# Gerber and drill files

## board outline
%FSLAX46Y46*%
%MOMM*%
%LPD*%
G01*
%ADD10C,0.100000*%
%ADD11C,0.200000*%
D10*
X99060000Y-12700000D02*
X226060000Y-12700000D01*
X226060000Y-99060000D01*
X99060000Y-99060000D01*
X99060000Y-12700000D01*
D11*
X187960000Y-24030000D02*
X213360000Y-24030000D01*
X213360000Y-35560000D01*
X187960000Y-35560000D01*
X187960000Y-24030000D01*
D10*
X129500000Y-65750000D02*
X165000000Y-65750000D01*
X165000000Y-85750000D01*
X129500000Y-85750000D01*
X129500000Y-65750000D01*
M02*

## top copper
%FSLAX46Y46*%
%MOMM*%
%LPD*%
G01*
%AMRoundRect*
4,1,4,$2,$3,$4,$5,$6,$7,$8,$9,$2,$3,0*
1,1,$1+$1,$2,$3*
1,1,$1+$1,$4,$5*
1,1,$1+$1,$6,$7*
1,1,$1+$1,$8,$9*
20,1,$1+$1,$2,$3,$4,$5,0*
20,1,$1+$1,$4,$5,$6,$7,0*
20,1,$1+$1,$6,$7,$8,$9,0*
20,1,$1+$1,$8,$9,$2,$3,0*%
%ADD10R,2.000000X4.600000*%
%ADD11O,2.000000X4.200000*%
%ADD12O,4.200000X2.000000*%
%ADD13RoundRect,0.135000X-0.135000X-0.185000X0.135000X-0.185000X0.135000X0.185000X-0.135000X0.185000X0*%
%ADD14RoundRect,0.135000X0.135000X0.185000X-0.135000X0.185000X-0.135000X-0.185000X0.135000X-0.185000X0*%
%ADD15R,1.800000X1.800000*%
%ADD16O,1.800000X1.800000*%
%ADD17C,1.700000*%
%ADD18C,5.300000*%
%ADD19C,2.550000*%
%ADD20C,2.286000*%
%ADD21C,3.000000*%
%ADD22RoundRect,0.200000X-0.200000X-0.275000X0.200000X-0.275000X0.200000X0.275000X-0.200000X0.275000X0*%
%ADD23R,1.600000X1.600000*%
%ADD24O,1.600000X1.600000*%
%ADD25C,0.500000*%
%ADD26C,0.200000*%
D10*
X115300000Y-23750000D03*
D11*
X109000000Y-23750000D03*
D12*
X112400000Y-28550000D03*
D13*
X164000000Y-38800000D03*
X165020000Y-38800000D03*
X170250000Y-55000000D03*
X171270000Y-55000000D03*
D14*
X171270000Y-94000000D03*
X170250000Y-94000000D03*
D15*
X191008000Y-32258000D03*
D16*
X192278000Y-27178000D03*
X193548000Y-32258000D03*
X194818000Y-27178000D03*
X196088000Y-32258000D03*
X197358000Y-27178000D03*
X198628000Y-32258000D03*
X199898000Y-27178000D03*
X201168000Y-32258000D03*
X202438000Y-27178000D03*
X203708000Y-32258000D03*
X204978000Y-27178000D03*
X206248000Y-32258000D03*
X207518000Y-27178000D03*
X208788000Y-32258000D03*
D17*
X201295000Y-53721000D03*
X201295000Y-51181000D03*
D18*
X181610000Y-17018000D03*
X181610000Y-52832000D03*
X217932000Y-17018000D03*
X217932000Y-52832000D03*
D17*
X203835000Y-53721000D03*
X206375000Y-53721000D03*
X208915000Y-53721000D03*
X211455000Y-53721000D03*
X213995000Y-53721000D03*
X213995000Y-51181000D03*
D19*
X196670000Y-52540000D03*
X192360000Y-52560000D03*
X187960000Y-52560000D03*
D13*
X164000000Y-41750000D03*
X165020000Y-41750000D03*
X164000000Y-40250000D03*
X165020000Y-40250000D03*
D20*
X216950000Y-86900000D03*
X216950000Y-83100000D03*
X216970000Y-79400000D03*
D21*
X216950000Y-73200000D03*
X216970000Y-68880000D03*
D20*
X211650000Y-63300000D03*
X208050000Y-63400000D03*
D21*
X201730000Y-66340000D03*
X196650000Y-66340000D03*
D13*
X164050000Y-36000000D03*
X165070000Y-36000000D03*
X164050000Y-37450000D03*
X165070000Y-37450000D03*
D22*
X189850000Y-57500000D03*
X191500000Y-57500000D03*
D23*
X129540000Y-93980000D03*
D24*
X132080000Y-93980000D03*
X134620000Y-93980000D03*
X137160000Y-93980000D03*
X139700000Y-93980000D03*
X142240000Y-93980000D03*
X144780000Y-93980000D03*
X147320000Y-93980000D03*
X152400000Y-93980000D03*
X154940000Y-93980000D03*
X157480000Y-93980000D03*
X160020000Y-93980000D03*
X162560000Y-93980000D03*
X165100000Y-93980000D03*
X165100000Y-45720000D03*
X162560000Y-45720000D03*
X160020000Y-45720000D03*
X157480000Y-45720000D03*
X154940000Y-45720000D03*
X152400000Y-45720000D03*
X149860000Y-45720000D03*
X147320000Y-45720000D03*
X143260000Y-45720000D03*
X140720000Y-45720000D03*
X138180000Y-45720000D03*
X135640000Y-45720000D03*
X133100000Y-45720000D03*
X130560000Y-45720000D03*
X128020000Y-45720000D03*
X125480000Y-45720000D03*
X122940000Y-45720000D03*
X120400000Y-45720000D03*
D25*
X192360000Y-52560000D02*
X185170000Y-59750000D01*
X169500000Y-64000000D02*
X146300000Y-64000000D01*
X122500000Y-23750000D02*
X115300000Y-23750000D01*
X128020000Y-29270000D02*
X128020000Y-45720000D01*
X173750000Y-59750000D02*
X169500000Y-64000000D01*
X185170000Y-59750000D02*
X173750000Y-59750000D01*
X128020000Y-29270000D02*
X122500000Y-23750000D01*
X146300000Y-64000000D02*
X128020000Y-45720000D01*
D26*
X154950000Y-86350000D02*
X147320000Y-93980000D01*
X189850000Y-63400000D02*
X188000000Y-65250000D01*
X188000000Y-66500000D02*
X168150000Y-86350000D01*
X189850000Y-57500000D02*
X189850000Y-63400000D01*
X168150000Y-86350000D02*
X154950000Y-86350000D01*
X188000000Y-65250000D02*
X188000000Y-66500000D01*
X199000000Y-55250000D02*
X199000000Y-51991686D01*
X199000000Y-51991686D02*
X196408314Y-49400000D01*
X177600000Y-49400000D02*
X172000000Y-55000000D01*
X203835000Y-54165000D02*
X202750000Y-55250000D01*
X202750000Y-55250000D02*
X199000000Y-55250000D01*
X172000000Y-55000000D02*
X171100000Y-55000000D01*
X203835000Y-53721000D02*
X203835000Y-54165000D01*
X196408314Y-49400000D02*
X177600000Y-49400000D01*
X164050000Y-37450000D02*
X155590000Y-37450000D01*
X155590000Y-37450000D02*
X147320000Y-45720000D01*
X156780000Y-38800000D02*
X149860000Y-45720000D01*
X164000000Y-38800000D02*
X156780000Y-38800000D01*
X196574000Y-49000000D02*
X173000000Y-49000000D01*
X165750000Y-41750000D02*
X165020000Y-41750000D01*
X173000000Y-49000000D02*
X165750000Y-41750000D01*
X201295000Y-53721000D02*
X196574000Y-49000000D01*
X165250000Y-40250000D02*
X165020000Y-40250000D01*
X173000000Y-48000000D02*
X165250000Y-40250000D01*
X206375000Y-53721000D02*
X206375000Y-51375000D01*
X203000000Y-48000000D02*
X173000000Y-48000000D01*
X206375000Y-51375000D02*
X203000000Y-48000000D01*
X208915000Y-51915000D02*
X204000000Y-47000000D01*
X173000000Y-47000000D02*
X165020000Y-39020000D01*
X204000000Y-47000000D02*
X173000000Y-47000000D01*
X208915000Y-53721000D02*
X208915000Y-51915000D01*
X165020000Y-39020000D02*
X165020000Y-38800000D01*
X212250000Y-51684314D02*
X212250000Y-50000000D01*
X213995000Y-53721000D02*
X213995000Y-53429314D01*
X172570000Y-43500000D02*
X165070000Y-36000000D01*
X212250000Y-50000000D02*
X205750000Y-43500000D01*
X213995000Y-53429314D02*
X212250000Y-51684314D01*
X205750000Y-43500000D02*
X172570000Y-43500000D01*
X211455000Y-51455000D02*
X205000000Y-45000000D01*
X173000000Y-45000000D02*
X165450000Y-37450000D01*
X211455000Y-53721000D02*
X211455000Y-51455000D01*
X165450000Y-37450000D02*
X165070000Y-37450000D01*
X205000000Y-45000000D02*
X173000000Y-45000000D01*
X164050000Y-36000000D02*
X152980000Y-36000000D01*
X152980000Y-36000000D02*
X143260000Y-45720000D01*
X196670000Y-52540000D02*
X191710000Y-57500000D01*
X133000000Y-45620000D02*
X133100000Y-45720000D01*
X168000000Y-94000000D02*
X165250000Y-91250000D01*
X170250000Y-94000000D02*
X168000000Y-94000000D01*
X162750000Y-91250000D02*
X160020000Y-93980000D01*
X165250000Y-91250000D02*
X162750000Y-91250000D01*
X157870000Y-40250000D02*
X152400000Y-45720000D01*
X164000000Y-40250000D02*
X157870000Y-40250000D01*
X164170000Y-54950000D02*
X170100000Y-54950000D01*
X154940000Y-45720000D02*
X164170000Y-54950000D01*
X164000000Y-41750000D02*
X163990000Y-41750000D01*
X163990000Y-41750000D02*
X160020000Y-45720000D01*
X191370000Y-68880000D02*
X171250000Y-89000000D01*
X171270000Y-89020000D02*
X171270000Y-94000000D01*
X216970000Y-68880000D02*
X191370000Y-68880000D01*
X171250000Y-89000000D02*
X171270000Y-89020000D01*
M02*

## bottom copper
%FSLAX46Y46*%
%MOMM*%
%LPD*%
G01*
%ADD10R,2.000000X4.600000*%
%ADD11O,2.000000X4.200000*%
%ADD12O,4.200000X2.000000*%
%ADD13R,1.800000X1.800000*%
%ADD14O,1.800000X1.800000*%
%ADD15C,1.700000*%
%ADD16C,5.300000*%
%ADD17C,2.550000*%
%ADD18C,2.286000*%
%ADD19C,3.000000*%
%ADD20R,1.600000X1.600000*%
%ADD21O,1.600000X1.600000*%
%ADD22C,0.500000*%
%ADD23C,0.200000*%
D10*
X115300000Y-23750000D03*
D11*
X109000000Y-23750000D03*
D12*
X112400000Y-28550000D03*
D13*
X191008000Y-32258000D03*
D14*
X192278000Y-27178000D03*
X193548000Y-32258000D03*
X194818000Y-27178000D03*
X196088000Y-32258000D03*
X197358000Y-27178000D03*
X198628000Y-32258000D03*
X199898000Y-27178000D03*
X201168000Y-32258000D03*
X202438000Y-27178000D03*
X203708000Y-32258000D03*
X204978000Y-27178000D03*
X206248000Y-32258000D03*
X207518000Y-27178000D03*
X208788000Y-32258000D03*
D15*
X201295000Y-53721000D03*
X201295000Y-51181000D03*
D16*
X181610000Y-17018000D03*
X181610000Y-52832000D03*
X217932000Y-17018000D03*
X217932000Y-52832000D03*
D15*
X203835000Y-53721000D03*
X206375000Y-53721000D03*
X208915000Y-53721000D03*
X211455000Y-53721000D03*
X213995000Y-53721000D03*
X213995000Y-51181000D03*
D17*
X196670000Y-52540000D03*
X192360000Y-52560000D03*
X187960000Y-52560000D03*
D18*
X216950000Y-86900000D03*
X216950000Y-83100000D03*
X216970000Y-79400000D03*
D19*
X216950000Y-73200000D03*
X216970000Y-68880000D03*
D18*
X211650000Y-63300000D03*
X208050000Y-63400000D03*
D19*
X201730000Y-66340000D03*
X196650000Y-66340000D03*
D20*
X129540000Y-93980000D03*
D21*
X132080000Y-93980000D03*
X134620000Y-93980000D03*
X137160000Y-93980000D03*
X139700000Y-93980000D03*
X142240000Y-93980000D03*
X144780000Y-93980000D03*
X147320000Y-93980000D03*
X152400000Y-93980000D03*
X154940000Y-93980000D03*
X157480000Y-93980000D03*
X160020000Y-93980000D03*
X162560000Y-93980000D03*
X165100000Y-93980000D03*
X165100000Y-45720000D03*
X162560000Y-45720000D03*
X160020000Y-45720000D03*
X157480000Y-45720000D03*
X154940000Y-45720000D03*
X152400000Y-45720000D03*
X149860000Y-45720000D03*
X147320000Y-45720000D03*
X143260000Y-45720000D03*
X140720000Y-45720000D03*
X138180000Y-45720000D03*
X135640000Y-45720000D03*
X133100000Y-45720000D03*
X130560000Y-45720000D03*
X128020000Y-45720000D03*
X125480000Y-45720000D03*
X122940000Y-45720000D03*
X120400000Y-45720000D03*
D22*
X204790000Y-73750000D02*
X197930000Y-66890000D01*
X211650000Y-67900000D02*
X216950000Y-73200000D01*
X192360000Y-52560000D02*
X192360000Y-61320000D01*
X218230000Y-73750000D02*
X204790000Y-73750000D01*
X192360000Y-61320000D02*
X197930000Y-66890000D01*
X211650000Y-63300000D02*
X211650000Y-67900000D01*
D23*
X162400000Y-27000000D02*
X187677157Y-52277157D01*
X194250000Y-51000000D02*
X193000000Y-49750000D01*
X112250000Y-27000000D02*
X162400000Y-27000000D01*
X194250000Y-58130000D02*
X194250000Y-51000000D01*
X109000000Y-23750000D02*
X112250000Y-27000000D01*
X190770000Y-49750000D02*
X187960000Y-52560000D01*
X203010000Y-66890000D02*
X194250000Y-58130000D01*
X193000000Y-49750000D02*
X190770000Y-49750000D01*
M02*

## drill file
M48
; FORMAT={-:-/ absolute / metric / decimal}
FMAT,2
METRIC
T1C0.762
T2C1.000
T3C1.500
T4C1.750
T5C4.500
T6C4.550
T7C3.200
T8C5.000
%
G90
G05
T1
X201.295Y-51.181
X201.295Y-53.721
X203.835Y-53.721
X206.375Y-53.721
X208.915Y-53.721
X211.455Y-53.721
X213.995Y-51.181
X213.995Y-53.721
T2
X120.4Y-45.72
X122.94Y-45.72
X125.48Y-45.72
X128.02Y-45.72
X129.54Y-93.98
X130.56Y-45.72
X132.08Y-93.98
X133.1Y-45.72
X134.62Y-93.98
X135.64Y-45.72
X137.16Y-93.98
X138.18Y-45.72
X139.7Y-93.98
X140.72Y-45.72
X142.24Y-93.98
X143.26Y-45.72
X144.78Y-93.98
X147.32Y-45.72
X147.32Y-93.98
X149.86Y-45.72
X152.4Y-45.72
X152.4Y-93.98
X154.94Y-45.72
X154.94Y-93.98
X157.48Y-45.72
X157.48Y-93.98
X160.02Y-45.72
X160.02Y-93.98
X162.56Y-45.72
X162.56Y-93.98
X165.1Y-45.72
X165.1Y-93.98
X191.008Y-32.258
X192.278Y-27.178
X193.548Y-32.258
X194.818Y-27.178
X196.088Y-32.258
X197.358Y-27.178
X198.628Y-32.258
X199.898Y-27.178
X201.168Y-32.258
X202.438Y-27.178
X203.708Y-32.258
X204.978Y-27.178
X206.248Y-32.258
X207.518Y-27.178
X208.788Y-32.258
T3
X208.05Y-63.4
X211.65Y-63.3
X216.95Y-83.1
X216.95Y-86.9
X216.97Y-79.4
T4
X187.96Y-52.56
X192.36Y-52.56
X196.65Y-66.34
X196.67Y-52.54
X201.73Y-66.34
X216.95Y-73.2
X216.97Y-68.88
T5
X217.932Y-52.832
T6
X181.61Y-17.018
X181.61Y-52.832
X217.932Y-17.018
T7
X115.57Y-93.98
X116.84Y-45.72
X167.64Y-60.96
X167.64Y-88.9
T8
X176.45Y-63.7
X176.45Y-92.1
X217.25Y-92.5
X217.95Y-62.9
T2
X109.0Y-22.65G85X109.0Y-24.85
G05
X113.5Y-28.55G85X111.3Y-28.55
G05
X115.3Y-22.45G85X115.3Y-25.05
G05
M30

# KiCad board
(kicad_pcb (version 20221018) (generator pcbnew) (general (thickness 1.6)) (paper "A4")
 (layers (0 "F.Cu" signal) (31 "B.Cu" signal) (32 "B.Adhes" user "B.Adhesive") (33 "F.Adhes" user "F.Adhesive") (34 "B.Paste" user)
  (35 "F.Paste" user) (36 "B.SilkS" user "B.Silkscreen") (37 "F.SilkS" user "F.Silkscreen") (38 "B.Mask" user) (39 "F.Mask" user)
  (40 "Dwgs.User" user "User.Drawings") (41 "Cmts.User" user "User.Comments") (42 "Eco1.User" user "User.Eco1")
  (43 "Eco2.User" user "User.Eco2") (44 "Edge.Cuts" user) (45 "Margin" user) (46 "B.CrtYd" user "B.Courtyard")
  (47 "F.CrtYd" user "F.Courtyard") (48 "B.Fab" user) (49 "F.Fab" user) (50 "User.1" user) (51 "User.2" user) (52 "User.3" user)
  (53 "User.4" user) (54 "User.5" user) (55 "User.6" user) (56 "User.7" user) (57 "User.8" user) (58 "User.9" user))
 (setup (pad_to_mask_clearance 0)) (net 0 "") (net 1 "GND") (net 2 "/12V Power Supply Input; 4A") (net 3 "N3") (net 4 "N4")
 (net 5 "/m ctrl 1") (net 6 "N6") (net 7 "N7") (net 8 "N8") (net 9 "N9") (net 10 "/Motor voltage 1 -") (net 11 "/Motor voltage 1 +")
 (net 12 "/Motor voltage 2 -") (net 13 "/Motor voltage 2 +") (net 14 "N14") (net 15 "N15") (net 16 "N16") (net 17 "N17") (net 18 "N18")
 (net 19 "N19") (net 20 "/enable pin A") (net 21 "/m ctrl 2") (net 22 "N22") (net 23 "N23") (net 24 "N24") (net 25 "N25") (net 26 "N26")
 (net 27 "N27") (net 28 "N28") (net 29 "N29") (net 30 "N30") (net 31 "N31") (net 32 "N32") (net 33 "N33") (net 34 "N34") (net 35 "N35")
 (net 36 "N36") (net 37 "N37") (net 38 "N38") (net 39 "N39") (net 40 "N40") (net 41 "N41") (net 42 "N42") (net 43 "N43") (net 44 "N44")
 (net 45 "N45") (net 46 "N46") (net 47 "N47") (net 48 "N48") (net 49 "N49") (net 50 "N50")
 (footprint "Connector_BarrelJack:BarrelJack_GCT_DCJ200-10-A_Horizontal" (layer "F.Cu") (at 115.3 23.75 -90)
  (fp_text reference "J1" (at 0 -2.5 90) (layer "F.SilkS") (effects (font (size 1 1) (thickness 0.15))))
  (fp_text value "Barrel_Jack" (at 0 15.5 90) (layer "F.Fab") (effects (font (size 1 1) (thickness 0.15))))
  (pad "1" thru_hole rect (at 0 0 270) (size 4.6 2) (drill oval 3.6 1) (layers "*.Cu" "*.Mask") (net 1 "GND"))
  (pad "2" thru_hole oval (at 0 6.3 270) (size 4.2 2) (drill oval 3.2 1) (layers "*.Cu" "*.Mask") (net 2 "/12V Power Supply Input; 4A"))
  (pad "3" thru_hole oval (at 4.8 2.9 270) (size 2 4.2) (drill oval 1 3.2) (layers "*.Cu" "*.Mask")))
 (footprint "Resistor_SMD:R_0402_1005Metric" (layer "F.Cu") (at 164.51 38.8)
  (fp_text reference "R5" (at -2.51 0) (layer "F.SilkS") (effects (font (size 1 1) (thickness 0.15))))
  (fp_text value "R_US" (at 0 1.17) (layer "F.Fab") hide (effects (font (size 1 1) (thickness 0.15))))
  (pad "1" smd roundrect (at -0.51 0) (size 0.54 0.64) (layers "F.Cu" "F.Paste" "F.Mask") (roundrect_rratio 0.25) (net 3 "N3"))
  (pad "2" smd roundrect (at 0.51 0) (size 0.54 0.64) (layers "F.Cu" "F.Paste" "F.Mask") (roundrect_rratio 0.25) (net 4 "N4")))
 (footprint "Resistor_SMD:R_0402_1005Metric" (layer "F.Cu") (at 170.76 55)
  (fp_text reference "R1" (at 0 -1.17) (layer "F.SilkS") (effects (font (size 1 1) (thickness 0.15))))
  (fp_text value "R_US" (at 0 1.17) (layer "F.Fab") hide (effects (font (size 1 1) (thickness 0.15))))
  (pad "1" smd roundrect (at -0.51 0) (size 0.54 0.64) (layers "F.Cu" "F.Paste" "F.Mask") (roundrect_rratio 0.25) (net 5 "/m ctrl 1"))
  (pad "2" smd roundrect (at 0.51 0) (size 0.54 0.64) (layers "F.Cu" "F.Paste" "F.Mask") (roundrect_rratio 0.25) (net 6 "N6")))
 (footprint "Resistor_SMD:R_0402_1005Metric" (layer "F.Cu") (at 170.76 94 180)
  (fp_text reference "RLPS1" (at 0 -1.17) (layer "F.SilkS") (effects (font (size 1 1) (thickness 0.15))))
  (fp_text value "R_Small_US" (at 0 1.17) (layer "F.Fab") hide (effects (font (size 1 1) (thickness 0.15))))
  (pad "1" smd roundrect (at -0.51 0 180) (size 0.54 0.64) (layers "F.Cu" "F.Paste" "F.Mask") (roundrect_rratio 0.25) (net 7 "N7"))
  (pad "2" smd roundrect (at 0.51 0 180) (size 0.54 0.64) (layers "F.Cu" "F.Paste" "F.Mask") (roundrect_rratio 0.25) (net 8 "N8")))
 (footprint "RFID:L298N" (layer "F.Cu") (at 200.66 35.56)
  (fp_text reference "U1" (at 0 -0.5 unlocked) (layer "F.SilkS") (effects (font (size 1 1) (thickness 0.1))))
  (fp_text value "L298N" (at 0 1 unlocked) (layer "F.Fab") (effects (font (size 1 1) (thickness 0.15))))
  (pad "1" thru_hole rect (at -9.652 -3.302) (size 1.8 1.8) (drill 1) (layers "*.Cu" "*.Mask") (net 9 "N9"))
  (pad "2" thru_hole oval (at -8.382 -8.382) (size 1.8 1.8) (drill 1) (layers "*.Cu" "*.Mask") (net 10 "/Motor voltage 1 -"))
  (pad "3" thru_hole oval (at -7.112 -3.302) (size 1.8 1.8) (drill 1) (layers "*.Cu" "*.Mask") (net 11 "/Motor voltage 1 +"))
  (pad "4" thru_hole oval (at -5.842 -8.382) (size 1.8 1.8) (drill 1) (layers "*.Cu" "*.Mask"))
  (pad "5" thru_hole oval (at -4.572 -3.302) (size 1.8 1.8) (drill 1) (layers "*.Cu" "*.Mask"))
  (pad "6" thru_hole oval (at -3.302 -8.382) (size 1.8 1.8) (drill 1) (layers "*.Cu" "*.Mask"))
  (pad "7" thru_hole oval (at -2.032 -3.302) (size 1.8 1.8) (drill 1) (layers "*.Cu" "*.Mask"))
  (pad "8" thru_hole oval (at -0.762 -8.382) (size 1.8 1.8) (drill 1) (layers "*.Cu" "*.Mask"))
  (pad "9" thru_hole oval (at 0.508 -3.302) (size 1.8 1.8) (drill 1) (layers "*.Cu" "*.Mask"))
  (pad "10" thru_hole oval (at 1.778 -8.382) (size 1.8 1.8) (drill 1) (layers "*.Cu" "*.Mask"))
  (pad "11" thru_hole oval (at 3.048 -3.302) (size 1.8 1.8) (drill 1) (layers "*.Cu" "*.Mask"))
  (pad "12" thru_hole oval (at 4.318 -8.382) (size 1.8 1.8) (drill 1) (layers "*.Cu" "*.Mask"))
  (pad "13" thru_hole oval (at 5.588 -3.302) (size 1.8 1.8) (drill 1) (layers "*.Cu" "*.Mask") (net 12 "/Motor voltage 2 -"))
  (pad "14" thru_hole oval (at 6.858 -8.382) (size 1.8 1.8) (drill 1) (layers "*.Cu" "*.Mask") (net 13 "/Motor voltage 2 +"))
  (pad "15" thru_hole oval (at 8.128 -3.302) (size 1.8 1.8) (drill 1) (layers "*.Cu" "*.Mask") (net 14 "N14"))
  (pad "23" thru_hole circle (at 0.635 18.161) (size 1.7 1.7) (drill 0.762) (layers "*.Cu" "*.Mask") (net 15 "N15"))
  (pad "24" thru_hole circle (at 0.635 15.621) (size 1.7 1.7) (drill 0.762) (layers "*.Cu" "*.Mask"))
  (pad "25" thru_hole circle (at -19.05 -18.542) (size 5.3 5.3) (drill 4.55) (layers "*.Cu" "*.Mask"))
  (pad "25" thru_hole circle (at -19.05 17.272) (size 5.3 5.3) (drill 4.55) (layers "*.Cu" "*.Mask"))
  (pad "25" thru_hole circle (at 17.272 -18.542) (size 5.3 5.3) (drill 4.55) (layers "*.Cu" "*.Mask"))
  (pad "25" thru_hole circle (at 17.272 17.272) (size 5.3 5.3) (drill 4.5) (layers "*.Cu" "*.Mask"))
  (pad "26" thru_hole circle (at 3.175 18.161) (size 1.7 1.7) (drill 0.762) (layers "*.Cu" "*.Mask") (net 6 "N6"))
  (pad "27" thru_hole circle (at 5.715 18.161) (size 1.7 1.7) (drill 0.762) (layers "*.Cu" "*.Mask") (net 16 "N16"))
  (pad "28" thru_hole circle (at 8.255 18.161) (size 1.7 1.7) (drill 0.762) (layers "*.Cu" "*.Mask") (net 4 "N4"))
  (pad "29" thru_hole circle (at 10.795 18.161) (size 1.7 1.7) (drill 0.762) (layers "*.Cu" "*.Mask") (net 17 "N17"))
  (pad "30" thru_hole circle (at 13.335 18.161) (size 1.7 1.7) (drill 0.762) (layers "*.Cu" "*.Mask") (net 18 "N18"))
  (pad "31" thru_hole circle (at 13.335 15.621) (size 1.7 1.7) (drill 0.762) (layers "*.Cu" "*.Mask"))
  (pad "32" thru_hole circle (at -3.99 16.98) (size 2.55 2.55) (drill 1.75) (layers "*.Cu" "*.Mask") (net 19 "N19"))
  (pad "33" thru_hole circle (at -8.3 17) (size 2.55 2.55) (drill 1.75) (layers "*.Cu" "*.Mask") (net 1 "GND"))
  (pad "34" thru_hole circle (at -12.7 17) (size 2.55 2.55) (drill 1.75) (layers "*.Cu" "*.Mask") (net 2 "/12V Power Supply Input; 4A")))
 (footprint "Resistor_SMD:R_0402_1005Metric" (layer "F.Cu") (at 164.51 41.75)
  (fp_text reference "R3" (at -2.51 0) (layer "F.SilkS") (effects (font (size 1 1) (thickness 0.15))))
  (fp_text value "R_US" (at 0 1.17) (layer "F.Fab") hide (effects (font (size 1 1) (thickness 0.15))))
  (pad "1" smd roundrect (at -0.51 0) (size 0.54 0.64) (layers "F.Cu" "F.Paste" "F.Mask") (roundrect_rratio 0.25) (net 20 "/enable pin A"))
  (pad "2" smd roundrect (at 0.51 0) (size 0.54 0.64) (layers "F.Cu" "F.Paste" "F.Mask") (roundrect_rratio 0.25) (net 15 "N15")))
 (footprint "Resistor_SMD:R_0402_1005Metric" (layer "F.Cu") (at 164.51 40.25)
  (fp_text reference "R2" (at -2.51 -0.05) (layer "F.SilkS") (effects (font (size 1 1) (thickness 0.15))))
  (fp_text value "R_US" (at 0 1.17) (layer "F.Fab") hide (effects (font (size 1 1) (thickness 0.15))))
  (pad "1" smd roundrect (at -0.51 0) (size 0.54 0.64) (layers "F.Cu" "F.Paste" "F.Mask") (roundrect_rratio 0.25) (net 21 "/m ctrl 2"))
  (pad "2" smd roundrect (at 0.51 0) (size 0.54 0.64) (layers "F.Cu" "F.Paste" "F.Mask") (roundrect_rratio 0.25) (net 16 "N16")))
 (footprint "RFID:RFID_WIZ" (layer "F.Cu") (at 196.65 76.5)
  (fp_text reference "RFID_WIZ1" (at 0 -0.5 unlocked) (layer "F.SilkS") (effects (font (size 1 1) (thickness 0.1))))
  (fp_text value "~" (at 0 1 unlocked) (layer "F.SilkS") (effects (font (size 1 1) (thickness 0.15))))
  (pad "" np_thru_hole circle (at -20.2 -12.8) (size 5 5) (drill 5) (layers "F&B.Cu" "*.Mask"))
  (pad "" np_thru_hole circle (at -20.2 15.6) (size 5 5) (drill 5) (layers "F&B.Cu" "*.Mask"))
  (pad "" np_thru_hole circle (at 20.6 16) (size 5 5) (drill 5) (layers "F&B.Cu" "*.Mask"))
  (pad "" np_thru_hole circle (at 21.3 -13.6) (size 5 5) (drill 5) (layers "F&B.Cu" "*.Mask"))
  (pad "1" thru_hole circle (at 20.3 10.4) (size 2.286 2.286) (drill 1.5) (layers "*.Cu" "*.Mask") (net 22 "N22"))
  (pad "2" thru_hole circle (at 20.3 6.6) (size 2.286 2.286) (drill 1.5) (layers "*.Cu" "*.Mask") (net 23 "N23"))
  (pad "3" thru_hole circle (at 20.32 2.9) (size 2.286 2.286) (drill 1.5) (layers "*.Cu" "*.Mask") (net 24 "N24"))
  (pad "4" thru_hole circle (at 20.3 -3.3) (size 3 3) (drill 1.75) (layers "*.Cu" "*.Mask") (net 1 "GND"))
  (pad "5" thru_hole circle (at 20.32 -7.62) (size 3 3) (drill 1.75) (layers "*.Cu" "*.Mask") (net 7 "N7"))
  (pad "6" thru_hole circle (at 15 -13.2) (size 2.286 2.286) (drill 1.5) (layers "*.Cu" "*.Mask") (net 1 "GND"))
  (pad "7" thru_hole circle (at 11.4 -13.1) (size 2.286 2.286) (drill 1.5) (layers "*.Cu" "*.Mask"))
  (pad "8" thru_hole circle (at 5.08 -10.16) (size 3 3) (drill 1.75) (layers "*.Cu" "*.Mask") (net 2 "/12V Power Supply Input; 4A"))
  (pad "9" thru_hole circle (at 0 -10.16) (size 3 3) (drill 1.75) (layers "*.Cu" "*.Mask") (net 1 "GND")))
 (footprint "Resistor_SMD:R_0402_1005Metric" (layer "F.Cu") (at 164.56 36)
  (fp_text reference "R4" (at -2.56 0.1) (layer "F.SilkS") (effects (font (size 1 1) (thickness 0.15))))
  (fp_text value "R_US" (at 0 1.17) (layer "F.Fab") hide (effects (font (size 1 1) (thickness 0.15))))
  (pad "1" smd roundrect (at -0.51 0) (size 0.54 0.64) (layers "F.Cu" "F.Paste" "F.Mask") (roundrect_rratio 0.25) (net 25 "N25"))
  (pad "2" smd roundrect (at 0.51 0) (size 0.54 0.64) (layers "F.Cu" "F.Paste" "F.Mask") (roundrect_rratio 0.25) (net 18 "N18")))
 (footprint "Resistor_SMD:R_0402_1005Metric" (layer "F.Cu") (at 164.56 37.45)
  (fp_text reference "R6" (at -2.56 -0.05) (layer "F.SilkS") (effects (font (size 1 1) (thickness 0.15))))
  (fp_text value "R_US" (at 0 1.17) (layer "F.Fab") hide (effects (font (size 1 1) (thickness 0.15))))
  (pad "1" smd roundrect (at -0.51 0) (size 0.54 0.64) (layers "F.Cu" "F.Paste" "F.Mask") (roundrect_rratio 0.25) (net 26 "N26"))
  (pad "2" smd roundrect (at 0.51 0) (size 0.54 0.64) (layers "F.Cu" "F.Paste" "F.Mask") (roundrect_rratio 0.25) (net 17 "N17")))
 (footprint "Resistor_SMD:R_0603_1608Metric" (layer "F.Cu") (at 190.675 57.5)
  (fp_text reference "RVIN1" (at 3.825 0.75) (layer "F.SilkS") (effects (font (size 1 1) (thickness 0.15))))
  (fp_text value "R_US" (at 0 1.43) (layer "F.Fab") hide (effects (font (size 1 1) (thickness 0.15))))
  (pad "1" smd roundrect (at -0.825 0) (size 0.8 0.95) (layers "F.Cu" "F.Paste" "F.Mask") (roundrect_rratio 0.25) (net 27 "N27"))
  (pad "2" smd roundrect (at 0.825 0) (size 0.8 0.95) (layers "F.Cu" "F.Paste" "F.Mask") (roundrect_rratio 0.25) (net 19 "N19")))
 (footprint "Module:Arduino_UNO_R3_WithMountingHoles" (layer "B.Cu") (at 129.54 93.98)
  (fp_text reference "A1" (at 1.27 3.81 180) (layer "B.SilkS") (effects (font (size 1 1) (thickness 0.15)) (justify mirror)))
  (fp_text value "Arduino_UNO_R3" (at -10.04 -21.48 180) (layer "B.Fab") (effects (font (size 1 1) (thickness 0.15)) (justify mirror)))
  (pad "" np_thru_hole circle (at -13.97 0 270) (size 3.2 3.2) (drill 3.2) (layers "*.Cu" "*.Mask"))
  (pad "" np_thru_hole circle (at -12.7 -48.26 270) (size 3.2 3.2) (drill 3.2) (layers "*.Cu" "*.Mask"))
  (pad "" np_thru_hole circle (at 38.1 -33.02 270) (size 3.2 3.2) (drill 3.2) (layers "*.Cu" "*.Mask"))
  (pad "" np_thru_hole circle (at 38.1 -5.08 270) (size 3.2 3.2) (drill 3.2) (layers "*.Cu" "*.Mask"))
  (pad "1" thru_hole rect (at 0 0 270) (size 1.6 1.6) (drill 1) (layers "*.Cu" "*.Mask") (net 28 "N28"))
  (pad "2" thru_hole oval (at 2.54 0 270) (size 1.6 1.6) (drill 1) (layers "*.Cu" "*.Mask") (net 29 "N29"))
  (pad "3" thru_hole oval (at 5.08 0 270) (size 1.6 1.6) (drill 1) (layers "*.Cu" "*.Mask") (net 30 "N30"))
  (pad "4" thru_hole oval (at 7.62 0 270) (size 1.6 1.6) (drill 1) (layers "*.Cu" "*.Mask") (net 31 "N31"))
  (pad "5" thru_hole oval (at 10.16 0 270) (size 1.6 1.6) (drill 1) (layers "*.Cu" "*.Mask") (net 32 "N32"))
  (pad "6" thru_hole oval (at 12.7 0 270) (size 1.6 1.6) (drill 1) (layers "*.Cu" "*.Mask") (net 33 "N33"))
  (pad "7" thru_hole oval (at 15.24 0 270) (size 1.6 1.6) (drill 1) (layers "*.Cu" "*.Mask") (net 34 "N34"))
  (pad "8" thru_hole oval (at 17.78 0 270) (size 1.6 1.6) (drill 1) (layers "*.Cu" "*.Mask") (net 27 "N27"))
  (pad "9" thru_hole oval (at 22.86 0 270) (size 1.6 1.6) (drill 1) (layers "*.Cu" "*.Mask") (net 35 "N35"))
  (pad "10" thru_hole oval (at 25.4 0 270) (size 1.6 1.6) (drill 1) (layers "*.Cu" "*.Mask") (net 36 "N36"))
  (pad "11" thru_hole oval (at 27.94 0 270) (size 1.6 1.6) (drill 1) (layers "*.Cu" "*.Mask") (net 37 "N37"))
  (pad "12" thru_hole oval (at 30.48 0 270) (size 1.6 1.6) (drill 1) (layers "*.Cu" "*.Mask") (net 8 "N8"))
  (pad "13" thru_hole oval (at 33.02 0 270) (size 1.6 1.6) (drill 1) (layers "*.Cu" "*.Mask") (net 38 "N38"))
  (pad "14" thru_hole oval (at 35.56 0 270) (size 1.6 1.6) (drill 1) (layers "*.Cu" "*.Mask") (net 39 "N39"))
  (pad "15" thru_hole oval (at 35.56 -48.26 270) (size 1.6 1.6) (drill 1) (layers "*.Cu" "*.Mask") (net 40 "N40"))
  (pad "16" thru_hole oval (at 33.02 -48.26 270) (size 1.6 1.6) (drill 1) (layers "*.Cu" "*.Mask") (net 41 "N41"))
  (pad "17" thru_hole oval (at 30.48 -48.26 270) (size 1.6 1.6) (drill 1) (layers "*.Cu" "*.Mask") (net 20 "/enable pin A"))
  (pad "18" thru_hole oval (at 27.94 -48.26 270) (size 1.6 1.6) (drill 1) (layers "*.Cu" "*.Mask") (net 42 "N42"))
  (pad "19" thru_hole oval (at 25.4 -48.26 270) (size 1.6 1.6) (drill 1) (layers "*.Cu" "*.Mask") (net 5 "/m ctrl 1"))
  (pad "20" thru_hole oval (at 22.86 -48.26 270) (size 1.6 1.6) (drill 1) (layers "*.Cu" "*.Mask") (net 21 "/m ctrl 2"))
  (pad "21" thru_hole oval (at 20.32 -48.26 270) (size 1.6 1.6) (drill 1) (layers "*.Cu" "*.Mask") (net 3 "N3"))
  (pad "22" thru_hole oval (at 17.78 -48.26 270) (size 1.6 1.6) (drill 1) (layers "*.Cu" "*.Mask") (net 26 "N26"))
  (pad "23" thru_hole oval (at 13.72 -48.26 270) (size 1.6 1.6) (drill 1) (layers "*.Cu" "*.Mask") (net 25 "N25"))
  (pad "24" thru_hole oval (at 11.18 -48.26 270) (size 1.6 1.6) (drill 1) (layers "*.Cu" "*.Mask") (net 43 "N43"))
  (pad "25" thru_hole oval (at 8.64 -48.26 270) (size 1.6 1.6) (drill 1) (layers "*.Cu" "*.Mask") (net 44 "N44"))
  (pad "26" thru_hole oval (at 6.1 -48.26 270) (size 1.6 1.6) (drill 1) (layers "*.Cu" "*.Mask") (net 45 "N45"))
  (pad "27" thru_hole oval (at 3.56 -48.26 270) (size 1.6 1.6) (drill 1) (layers "*.Cu" "*.Mask") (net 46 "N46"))
  (pad "28" thru_hole oval (at 1.02 -48.26 270) (size 1.6 1.6) (drill 1) (layers "*.Cu" "*.Mask") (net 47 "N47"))
  (pad "29" thru_hole oval (at -1.52 -48.26 270) (size 1.6 1.6) (drill 1) (layers "*.Cu" "*.Mask") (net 1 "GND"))
  (pad "30" thru_hole oval (at -4.06 -48.26 270) (size 1.6 1.6) (drill 1) (layers "*.Cu" "*.Mask") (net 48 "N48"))
  (pad "31" thru_hole oval (at -6.6 -48.26 270) (size 1.6 1.6) (drill 1) (layers "*.Cu" "*.Mask") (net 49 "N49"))
  (pad "32" thru_hole oval (at -9.14 -48.26 270) (size 1.6 1.6) (drill 1) (layers "*.Cu" "*.Mask") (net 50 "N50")))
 (gr_rect (start 99.06 12.7) (end 226.06 99.06) (stroke (width 0.1) (type default)) (fill none) (layer "Edge.Cuts"))
 (gr_rect (start 187.96 24.03) (end 213.36 35.56) (stroke (width 0.2) (type default)) (fill none) (layer "Edge.Cuts"))
 (gr_rect (start 129.5 65.75) (end 165 85.75) (stroke (width 0.1) (type default)) (fill none) (layer "Edge.Cuts"))
 (segment (start 192.36 52.56) (end 185.17 59.75) (width 0.5) (layer "F.Cu") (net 1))
 (segment (start 169.5 64) (end 146.3 64) (width 0.5) (layer "F.Cu") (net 1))
 (segment (start 122.5 23.75) (end 115.3 23.75) (width 0.5) (layer "F.Cu") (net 1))
 (segment (start 128.02 29.27) (end 128.02 45.72) (width 0.5) (layer "F.Cu") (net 1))
 (segment (start 173.75 59.75) (end 169.5 64) (width 0.5) (layer "F.Cu") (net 1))
 (segment (start 185.17 59.75) (end 173.75 59.75) (width 0.5) (layer "F.Cu") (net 1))
 (segment (start 128.02 29.27) (end 122.5 23.75) (width 0.5) (layer "F.Cu") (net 1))
 (segment (start 146.3 64) (end 128.02 45.72) (width 0.5) (layer "F.Cu") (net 1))
 (segment (start 204.79 73.75) (end 197.93 66.89) (width 0.5) (layer "B.Cu") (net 1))
 (segment (start 211.65 67.9) (end 216.95 73.2) (width 0.5) (layer "B.Cu") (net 1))
 (segment (start 192.36 52.56) (end 192.36 61.32) (width 0.5) (layer "B.Cu") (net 1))
 (segment (start 218.23 73.75) (end 204.79 73.75) (width 0.5) (layer "B.Cu") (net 1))
 (segment (start 192.36 61.32) (end 197.93 66.89) (width 0.5) (layer "B.Cu") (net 1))
 (segment (start 211.65 63.3) (end 211.65 67.9) (width 0.5) (layer "B.Cu") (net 1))
 (segment (start 154.95 86.35) (end 147.32 93.98) (width 0.2) (layer "F.Cu") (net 27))
 (segment (start 189.85 63.4) (end 188 65.25) (width 0.2) (layer "F.Cu") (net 27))
 (segment (start 188 66.5) (end 168.15 86.35) (width 0.2) (layer "F.Cu") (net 27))
 (segment (start 189.85 57.5) (end 189.85 63.4) (width 0.2) (layer "F.Cu") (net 27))
 (segment (start 168.15 86.35) (end 154.95 86.35) (width 0.2) (layer "F.Cu") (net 27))
 (segment (start 188 65.25) (end 188 66.5) (width 0.2) (layer "F.Cu") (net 27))
 (segment (start 199 55.25) (end 199 51.991686) (width 0.2) (layer "F.Cu") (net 6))
 (segment (start 199 51.991686) (end 196.408314 49.4) (width 0.2) (layer "F.Cu") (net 6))
 (segment (start 177.6 49.4) (end 172 55) (width 0.2) (layer "F.Cu") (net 6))
 (segment (start 203.835 54.165) (end 202.75 55.25) (width 0.2) (layer "F.Cu") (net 6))
 (segment (start 202.75 55.25) (end 199 55.25) (width 0.2) (layer "F.Cu") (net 6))
 (segment (start 172 55) (end 171.1 55) (width 0.2) (layer "F.Cu") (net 6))
 (segment (start 203.835 53.721) (end 203.835 54.165) (width 0.2) (layer "F.Cu") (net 6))
 (segment (start 196.408314 49.4) (end 177.6 49.4) (width 0.2) (layer "F.Cu") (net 6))
 (segment (start 164.05 37.45) (end 155.59 37.45) (width 0.2) (layer "F.Cu") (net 26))
 (segment (start 155.59 37.45) (end 147.32 45.72) (width 0.2) (layer "F.Cu") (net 26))
 (segment (start 156.78 38.8) (end 149.86 45.72) (width 0.2) (layer "F.Cu") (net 3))
 (segment (start 164 38.8) (end 156.78 38.8) (width 0.2) (layer "F.Cu") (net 3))
 (segment (start 196.574 49) (end 173 49) (width 0.2) (layer "F.Cu") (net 15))
 (segment (start 165.75 41.75) (end 165.02 41.75) (width 0.2) (layer "F.Cu") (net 15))
 (segment (start 173 49) (end 165.75 41.75) (width 0.2) (layer "F.Cu") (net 15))
 (segment (start 201.295 53.721) (end 196.574 49) (width 0.2) (layer "F.Cu") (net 15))
 (segment (start 165.25 40.25) (end 165.02 40.25) (width 0.2) (layer "F.Cu") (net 16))
 (segment (start 173 48) (end 165.25 40.25) (width 0.2) (layer "F.Cu") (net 16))
 (segment (start 206.375 53.721) (end 206.375 51.375) (width 0.2) (layer "F.Cu") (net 16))
 (segment (start 203 48) (end 173 48) (width 0.2) (layer "F.Cu") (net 16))
 (segment (start 206.375 51.375) (end 203 48) (width 0.2) (layer "F.Cu") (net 16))
 (segment (start 208.915 51.915) (end 204 47) (width 0.2) (layer "F.Cu") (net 4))
 (segment (start 173 47) (end 165.02 39.02) (width 0.2) (layer "F.Cu") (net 4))
 (segment (start 204 47) (end 173 47) (width 0.2) (layer "F.Cu") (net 4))
 (segment (start 208.915 53.721) (end 208.915 51.915) (width 0.2) (layer "F.Cu") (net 4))
 (segment (start 165.02 39.02) (end 165.02 38.8) (width 0.2) (layer "F.Cu") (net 4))
 (segment (start 212.25 51.684314) (end 212.25 50) (width 0.2) (layer "F.Cu") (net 18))
 (segment (start 213.995 53.721) (end 213.995 53.429314) (width 0.2) (layer "F.Cu") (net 18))
 (segment (start 172.57 43.5) (end 165.07 36) (width 0.2) (layer "F.Cu") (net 18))
 (segment (start 212.25 50) (end 205.75 43.5) (width 0.2) (layer "F.Cu") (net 18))
 (segment (start 213.995 53.429314) (end 212.25 51.684314) (width 0.2) (layer "F.Cu") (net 18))
 (segment (start 205.75 43.5) (end 172.57 43.5) (width 0.2) (layer "F.Cu") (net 18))
 (segment (start 211.455 51.455) (end 205 45) (width 0.2) (layer "F.Cu") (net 17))
 (segment (start 173 45) (end 165.45 37.45) (width 0.2) (layer "F.Cu") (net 17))
 (segment (start 211.455 53.721) (end 211.455 51.455) (width 0.2) (layer "F.Cu") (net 17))
 (segment (start 165.45 37.45) (end 165.07 37.45) (width 0.2) (layer "F.Cu") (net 17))
 (segment (start 205 45) (end 173 45) (width 0.2) (layer "F.Cu") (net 17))
 (segment (start 164.05 36) (end 152.98 36) (width 0.2) (layer "F.Cu") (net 25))
 (segment (start 152.98 36) (end 143.26 45.72) (width 0.2) (layer "F.Cu") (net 25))
 (segment (start 196.67 52.54) (end 191.71 57.5) (width 0.2) (layer "F.Cu") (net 19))
 (segment (start 133 45.62) (end 133.1 45.72) (width 0.2) (layer "F.Cu") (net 46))
 (segment (start 168 94) (end 165.25 91.25) (width 0.2) (layer "F.Cu") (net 8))
 (segment (start 170.25 94) (end 168 94) (width 0.2) (layer "F.Cu") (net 8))
 (segment (start 162.75 91.25) (end 160.02 93.98) (width 0.2) (layer "F.Cu") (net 8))
 (segment (start 165.25 91.25) (end 162.75 91.25) (width 0.2) (layer "F.Cu") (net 8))
 (segment (start 162.4 27) (end 187.677157 52.277157) (width 0.2) (layer "B.Cu") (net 2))
 (segment (start 194.25 51) (end 193 49.75) (width 0.2) (layer "B.Cu") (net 2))
 (segment (start 112.25 27) (end 162.4 27) (width 0.2) (layer "B.Cu") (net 2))
 (segment (start 194.25 58.13) (end 194.25 51) (width 0.2) (layer "B.Cu") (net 2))
 (segment (start 109 23.75) (end 112.25 27) (width 0.2) (layer "B.Cu") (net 2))
 (segment (start 190.77 49.75) (end 187.96 52.56) (width 0.2) (layer "B.Cu") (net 2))
 (segment (start 203.01 66.89) (end 194.25 58.13) (width 0.2) (layer "B.Cu") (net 2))
 (segment (start 193 49.75) (end 190.77 49.75) (width 0.2) (layer "B.Cu") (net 2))
 (segment (start 157.87 40.25) (end 152.4 45.72) (width 0.2) (layer "F.Cu") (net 21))
 (segment (start 164 40.25) (end 157.87 40.25) (width 0.2) (layer "F.Cu") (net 21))
 (segment (start 164.17 54.95) (end 170.1 54.95) (width 0.2) (layer "F.Cu") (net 5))
 (segment (start 154.94 45.72) (end 164.17 54.95) (width 0.2) (layer "F.Cu") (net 5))
 (segment (start 164 41.75) (end 163.99 41.75) (width 0.2) (layer "F.Cu") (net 20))
 (segment (start 163.99 41.75) (end 160.02 45.72) (width 0.2) (layer "F.Cu") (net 20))
 (segment (start 191.37 68.88) (end 171.25 89) (width 0.2) (layer "F.Cu") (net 7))
 (segment (start 171.27 89.02) (end 171.27 94) (width 0.2) (layer "F.Cu") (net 7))
 (segment (start 216.97 68.88) (end 191.37 68.88) (width 0.2) (layer "F.Cu") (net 7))
 (segment (start 171.25 89) (end 171.27 89.02) (width 0.2) (layer "F.Cu") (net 7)))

